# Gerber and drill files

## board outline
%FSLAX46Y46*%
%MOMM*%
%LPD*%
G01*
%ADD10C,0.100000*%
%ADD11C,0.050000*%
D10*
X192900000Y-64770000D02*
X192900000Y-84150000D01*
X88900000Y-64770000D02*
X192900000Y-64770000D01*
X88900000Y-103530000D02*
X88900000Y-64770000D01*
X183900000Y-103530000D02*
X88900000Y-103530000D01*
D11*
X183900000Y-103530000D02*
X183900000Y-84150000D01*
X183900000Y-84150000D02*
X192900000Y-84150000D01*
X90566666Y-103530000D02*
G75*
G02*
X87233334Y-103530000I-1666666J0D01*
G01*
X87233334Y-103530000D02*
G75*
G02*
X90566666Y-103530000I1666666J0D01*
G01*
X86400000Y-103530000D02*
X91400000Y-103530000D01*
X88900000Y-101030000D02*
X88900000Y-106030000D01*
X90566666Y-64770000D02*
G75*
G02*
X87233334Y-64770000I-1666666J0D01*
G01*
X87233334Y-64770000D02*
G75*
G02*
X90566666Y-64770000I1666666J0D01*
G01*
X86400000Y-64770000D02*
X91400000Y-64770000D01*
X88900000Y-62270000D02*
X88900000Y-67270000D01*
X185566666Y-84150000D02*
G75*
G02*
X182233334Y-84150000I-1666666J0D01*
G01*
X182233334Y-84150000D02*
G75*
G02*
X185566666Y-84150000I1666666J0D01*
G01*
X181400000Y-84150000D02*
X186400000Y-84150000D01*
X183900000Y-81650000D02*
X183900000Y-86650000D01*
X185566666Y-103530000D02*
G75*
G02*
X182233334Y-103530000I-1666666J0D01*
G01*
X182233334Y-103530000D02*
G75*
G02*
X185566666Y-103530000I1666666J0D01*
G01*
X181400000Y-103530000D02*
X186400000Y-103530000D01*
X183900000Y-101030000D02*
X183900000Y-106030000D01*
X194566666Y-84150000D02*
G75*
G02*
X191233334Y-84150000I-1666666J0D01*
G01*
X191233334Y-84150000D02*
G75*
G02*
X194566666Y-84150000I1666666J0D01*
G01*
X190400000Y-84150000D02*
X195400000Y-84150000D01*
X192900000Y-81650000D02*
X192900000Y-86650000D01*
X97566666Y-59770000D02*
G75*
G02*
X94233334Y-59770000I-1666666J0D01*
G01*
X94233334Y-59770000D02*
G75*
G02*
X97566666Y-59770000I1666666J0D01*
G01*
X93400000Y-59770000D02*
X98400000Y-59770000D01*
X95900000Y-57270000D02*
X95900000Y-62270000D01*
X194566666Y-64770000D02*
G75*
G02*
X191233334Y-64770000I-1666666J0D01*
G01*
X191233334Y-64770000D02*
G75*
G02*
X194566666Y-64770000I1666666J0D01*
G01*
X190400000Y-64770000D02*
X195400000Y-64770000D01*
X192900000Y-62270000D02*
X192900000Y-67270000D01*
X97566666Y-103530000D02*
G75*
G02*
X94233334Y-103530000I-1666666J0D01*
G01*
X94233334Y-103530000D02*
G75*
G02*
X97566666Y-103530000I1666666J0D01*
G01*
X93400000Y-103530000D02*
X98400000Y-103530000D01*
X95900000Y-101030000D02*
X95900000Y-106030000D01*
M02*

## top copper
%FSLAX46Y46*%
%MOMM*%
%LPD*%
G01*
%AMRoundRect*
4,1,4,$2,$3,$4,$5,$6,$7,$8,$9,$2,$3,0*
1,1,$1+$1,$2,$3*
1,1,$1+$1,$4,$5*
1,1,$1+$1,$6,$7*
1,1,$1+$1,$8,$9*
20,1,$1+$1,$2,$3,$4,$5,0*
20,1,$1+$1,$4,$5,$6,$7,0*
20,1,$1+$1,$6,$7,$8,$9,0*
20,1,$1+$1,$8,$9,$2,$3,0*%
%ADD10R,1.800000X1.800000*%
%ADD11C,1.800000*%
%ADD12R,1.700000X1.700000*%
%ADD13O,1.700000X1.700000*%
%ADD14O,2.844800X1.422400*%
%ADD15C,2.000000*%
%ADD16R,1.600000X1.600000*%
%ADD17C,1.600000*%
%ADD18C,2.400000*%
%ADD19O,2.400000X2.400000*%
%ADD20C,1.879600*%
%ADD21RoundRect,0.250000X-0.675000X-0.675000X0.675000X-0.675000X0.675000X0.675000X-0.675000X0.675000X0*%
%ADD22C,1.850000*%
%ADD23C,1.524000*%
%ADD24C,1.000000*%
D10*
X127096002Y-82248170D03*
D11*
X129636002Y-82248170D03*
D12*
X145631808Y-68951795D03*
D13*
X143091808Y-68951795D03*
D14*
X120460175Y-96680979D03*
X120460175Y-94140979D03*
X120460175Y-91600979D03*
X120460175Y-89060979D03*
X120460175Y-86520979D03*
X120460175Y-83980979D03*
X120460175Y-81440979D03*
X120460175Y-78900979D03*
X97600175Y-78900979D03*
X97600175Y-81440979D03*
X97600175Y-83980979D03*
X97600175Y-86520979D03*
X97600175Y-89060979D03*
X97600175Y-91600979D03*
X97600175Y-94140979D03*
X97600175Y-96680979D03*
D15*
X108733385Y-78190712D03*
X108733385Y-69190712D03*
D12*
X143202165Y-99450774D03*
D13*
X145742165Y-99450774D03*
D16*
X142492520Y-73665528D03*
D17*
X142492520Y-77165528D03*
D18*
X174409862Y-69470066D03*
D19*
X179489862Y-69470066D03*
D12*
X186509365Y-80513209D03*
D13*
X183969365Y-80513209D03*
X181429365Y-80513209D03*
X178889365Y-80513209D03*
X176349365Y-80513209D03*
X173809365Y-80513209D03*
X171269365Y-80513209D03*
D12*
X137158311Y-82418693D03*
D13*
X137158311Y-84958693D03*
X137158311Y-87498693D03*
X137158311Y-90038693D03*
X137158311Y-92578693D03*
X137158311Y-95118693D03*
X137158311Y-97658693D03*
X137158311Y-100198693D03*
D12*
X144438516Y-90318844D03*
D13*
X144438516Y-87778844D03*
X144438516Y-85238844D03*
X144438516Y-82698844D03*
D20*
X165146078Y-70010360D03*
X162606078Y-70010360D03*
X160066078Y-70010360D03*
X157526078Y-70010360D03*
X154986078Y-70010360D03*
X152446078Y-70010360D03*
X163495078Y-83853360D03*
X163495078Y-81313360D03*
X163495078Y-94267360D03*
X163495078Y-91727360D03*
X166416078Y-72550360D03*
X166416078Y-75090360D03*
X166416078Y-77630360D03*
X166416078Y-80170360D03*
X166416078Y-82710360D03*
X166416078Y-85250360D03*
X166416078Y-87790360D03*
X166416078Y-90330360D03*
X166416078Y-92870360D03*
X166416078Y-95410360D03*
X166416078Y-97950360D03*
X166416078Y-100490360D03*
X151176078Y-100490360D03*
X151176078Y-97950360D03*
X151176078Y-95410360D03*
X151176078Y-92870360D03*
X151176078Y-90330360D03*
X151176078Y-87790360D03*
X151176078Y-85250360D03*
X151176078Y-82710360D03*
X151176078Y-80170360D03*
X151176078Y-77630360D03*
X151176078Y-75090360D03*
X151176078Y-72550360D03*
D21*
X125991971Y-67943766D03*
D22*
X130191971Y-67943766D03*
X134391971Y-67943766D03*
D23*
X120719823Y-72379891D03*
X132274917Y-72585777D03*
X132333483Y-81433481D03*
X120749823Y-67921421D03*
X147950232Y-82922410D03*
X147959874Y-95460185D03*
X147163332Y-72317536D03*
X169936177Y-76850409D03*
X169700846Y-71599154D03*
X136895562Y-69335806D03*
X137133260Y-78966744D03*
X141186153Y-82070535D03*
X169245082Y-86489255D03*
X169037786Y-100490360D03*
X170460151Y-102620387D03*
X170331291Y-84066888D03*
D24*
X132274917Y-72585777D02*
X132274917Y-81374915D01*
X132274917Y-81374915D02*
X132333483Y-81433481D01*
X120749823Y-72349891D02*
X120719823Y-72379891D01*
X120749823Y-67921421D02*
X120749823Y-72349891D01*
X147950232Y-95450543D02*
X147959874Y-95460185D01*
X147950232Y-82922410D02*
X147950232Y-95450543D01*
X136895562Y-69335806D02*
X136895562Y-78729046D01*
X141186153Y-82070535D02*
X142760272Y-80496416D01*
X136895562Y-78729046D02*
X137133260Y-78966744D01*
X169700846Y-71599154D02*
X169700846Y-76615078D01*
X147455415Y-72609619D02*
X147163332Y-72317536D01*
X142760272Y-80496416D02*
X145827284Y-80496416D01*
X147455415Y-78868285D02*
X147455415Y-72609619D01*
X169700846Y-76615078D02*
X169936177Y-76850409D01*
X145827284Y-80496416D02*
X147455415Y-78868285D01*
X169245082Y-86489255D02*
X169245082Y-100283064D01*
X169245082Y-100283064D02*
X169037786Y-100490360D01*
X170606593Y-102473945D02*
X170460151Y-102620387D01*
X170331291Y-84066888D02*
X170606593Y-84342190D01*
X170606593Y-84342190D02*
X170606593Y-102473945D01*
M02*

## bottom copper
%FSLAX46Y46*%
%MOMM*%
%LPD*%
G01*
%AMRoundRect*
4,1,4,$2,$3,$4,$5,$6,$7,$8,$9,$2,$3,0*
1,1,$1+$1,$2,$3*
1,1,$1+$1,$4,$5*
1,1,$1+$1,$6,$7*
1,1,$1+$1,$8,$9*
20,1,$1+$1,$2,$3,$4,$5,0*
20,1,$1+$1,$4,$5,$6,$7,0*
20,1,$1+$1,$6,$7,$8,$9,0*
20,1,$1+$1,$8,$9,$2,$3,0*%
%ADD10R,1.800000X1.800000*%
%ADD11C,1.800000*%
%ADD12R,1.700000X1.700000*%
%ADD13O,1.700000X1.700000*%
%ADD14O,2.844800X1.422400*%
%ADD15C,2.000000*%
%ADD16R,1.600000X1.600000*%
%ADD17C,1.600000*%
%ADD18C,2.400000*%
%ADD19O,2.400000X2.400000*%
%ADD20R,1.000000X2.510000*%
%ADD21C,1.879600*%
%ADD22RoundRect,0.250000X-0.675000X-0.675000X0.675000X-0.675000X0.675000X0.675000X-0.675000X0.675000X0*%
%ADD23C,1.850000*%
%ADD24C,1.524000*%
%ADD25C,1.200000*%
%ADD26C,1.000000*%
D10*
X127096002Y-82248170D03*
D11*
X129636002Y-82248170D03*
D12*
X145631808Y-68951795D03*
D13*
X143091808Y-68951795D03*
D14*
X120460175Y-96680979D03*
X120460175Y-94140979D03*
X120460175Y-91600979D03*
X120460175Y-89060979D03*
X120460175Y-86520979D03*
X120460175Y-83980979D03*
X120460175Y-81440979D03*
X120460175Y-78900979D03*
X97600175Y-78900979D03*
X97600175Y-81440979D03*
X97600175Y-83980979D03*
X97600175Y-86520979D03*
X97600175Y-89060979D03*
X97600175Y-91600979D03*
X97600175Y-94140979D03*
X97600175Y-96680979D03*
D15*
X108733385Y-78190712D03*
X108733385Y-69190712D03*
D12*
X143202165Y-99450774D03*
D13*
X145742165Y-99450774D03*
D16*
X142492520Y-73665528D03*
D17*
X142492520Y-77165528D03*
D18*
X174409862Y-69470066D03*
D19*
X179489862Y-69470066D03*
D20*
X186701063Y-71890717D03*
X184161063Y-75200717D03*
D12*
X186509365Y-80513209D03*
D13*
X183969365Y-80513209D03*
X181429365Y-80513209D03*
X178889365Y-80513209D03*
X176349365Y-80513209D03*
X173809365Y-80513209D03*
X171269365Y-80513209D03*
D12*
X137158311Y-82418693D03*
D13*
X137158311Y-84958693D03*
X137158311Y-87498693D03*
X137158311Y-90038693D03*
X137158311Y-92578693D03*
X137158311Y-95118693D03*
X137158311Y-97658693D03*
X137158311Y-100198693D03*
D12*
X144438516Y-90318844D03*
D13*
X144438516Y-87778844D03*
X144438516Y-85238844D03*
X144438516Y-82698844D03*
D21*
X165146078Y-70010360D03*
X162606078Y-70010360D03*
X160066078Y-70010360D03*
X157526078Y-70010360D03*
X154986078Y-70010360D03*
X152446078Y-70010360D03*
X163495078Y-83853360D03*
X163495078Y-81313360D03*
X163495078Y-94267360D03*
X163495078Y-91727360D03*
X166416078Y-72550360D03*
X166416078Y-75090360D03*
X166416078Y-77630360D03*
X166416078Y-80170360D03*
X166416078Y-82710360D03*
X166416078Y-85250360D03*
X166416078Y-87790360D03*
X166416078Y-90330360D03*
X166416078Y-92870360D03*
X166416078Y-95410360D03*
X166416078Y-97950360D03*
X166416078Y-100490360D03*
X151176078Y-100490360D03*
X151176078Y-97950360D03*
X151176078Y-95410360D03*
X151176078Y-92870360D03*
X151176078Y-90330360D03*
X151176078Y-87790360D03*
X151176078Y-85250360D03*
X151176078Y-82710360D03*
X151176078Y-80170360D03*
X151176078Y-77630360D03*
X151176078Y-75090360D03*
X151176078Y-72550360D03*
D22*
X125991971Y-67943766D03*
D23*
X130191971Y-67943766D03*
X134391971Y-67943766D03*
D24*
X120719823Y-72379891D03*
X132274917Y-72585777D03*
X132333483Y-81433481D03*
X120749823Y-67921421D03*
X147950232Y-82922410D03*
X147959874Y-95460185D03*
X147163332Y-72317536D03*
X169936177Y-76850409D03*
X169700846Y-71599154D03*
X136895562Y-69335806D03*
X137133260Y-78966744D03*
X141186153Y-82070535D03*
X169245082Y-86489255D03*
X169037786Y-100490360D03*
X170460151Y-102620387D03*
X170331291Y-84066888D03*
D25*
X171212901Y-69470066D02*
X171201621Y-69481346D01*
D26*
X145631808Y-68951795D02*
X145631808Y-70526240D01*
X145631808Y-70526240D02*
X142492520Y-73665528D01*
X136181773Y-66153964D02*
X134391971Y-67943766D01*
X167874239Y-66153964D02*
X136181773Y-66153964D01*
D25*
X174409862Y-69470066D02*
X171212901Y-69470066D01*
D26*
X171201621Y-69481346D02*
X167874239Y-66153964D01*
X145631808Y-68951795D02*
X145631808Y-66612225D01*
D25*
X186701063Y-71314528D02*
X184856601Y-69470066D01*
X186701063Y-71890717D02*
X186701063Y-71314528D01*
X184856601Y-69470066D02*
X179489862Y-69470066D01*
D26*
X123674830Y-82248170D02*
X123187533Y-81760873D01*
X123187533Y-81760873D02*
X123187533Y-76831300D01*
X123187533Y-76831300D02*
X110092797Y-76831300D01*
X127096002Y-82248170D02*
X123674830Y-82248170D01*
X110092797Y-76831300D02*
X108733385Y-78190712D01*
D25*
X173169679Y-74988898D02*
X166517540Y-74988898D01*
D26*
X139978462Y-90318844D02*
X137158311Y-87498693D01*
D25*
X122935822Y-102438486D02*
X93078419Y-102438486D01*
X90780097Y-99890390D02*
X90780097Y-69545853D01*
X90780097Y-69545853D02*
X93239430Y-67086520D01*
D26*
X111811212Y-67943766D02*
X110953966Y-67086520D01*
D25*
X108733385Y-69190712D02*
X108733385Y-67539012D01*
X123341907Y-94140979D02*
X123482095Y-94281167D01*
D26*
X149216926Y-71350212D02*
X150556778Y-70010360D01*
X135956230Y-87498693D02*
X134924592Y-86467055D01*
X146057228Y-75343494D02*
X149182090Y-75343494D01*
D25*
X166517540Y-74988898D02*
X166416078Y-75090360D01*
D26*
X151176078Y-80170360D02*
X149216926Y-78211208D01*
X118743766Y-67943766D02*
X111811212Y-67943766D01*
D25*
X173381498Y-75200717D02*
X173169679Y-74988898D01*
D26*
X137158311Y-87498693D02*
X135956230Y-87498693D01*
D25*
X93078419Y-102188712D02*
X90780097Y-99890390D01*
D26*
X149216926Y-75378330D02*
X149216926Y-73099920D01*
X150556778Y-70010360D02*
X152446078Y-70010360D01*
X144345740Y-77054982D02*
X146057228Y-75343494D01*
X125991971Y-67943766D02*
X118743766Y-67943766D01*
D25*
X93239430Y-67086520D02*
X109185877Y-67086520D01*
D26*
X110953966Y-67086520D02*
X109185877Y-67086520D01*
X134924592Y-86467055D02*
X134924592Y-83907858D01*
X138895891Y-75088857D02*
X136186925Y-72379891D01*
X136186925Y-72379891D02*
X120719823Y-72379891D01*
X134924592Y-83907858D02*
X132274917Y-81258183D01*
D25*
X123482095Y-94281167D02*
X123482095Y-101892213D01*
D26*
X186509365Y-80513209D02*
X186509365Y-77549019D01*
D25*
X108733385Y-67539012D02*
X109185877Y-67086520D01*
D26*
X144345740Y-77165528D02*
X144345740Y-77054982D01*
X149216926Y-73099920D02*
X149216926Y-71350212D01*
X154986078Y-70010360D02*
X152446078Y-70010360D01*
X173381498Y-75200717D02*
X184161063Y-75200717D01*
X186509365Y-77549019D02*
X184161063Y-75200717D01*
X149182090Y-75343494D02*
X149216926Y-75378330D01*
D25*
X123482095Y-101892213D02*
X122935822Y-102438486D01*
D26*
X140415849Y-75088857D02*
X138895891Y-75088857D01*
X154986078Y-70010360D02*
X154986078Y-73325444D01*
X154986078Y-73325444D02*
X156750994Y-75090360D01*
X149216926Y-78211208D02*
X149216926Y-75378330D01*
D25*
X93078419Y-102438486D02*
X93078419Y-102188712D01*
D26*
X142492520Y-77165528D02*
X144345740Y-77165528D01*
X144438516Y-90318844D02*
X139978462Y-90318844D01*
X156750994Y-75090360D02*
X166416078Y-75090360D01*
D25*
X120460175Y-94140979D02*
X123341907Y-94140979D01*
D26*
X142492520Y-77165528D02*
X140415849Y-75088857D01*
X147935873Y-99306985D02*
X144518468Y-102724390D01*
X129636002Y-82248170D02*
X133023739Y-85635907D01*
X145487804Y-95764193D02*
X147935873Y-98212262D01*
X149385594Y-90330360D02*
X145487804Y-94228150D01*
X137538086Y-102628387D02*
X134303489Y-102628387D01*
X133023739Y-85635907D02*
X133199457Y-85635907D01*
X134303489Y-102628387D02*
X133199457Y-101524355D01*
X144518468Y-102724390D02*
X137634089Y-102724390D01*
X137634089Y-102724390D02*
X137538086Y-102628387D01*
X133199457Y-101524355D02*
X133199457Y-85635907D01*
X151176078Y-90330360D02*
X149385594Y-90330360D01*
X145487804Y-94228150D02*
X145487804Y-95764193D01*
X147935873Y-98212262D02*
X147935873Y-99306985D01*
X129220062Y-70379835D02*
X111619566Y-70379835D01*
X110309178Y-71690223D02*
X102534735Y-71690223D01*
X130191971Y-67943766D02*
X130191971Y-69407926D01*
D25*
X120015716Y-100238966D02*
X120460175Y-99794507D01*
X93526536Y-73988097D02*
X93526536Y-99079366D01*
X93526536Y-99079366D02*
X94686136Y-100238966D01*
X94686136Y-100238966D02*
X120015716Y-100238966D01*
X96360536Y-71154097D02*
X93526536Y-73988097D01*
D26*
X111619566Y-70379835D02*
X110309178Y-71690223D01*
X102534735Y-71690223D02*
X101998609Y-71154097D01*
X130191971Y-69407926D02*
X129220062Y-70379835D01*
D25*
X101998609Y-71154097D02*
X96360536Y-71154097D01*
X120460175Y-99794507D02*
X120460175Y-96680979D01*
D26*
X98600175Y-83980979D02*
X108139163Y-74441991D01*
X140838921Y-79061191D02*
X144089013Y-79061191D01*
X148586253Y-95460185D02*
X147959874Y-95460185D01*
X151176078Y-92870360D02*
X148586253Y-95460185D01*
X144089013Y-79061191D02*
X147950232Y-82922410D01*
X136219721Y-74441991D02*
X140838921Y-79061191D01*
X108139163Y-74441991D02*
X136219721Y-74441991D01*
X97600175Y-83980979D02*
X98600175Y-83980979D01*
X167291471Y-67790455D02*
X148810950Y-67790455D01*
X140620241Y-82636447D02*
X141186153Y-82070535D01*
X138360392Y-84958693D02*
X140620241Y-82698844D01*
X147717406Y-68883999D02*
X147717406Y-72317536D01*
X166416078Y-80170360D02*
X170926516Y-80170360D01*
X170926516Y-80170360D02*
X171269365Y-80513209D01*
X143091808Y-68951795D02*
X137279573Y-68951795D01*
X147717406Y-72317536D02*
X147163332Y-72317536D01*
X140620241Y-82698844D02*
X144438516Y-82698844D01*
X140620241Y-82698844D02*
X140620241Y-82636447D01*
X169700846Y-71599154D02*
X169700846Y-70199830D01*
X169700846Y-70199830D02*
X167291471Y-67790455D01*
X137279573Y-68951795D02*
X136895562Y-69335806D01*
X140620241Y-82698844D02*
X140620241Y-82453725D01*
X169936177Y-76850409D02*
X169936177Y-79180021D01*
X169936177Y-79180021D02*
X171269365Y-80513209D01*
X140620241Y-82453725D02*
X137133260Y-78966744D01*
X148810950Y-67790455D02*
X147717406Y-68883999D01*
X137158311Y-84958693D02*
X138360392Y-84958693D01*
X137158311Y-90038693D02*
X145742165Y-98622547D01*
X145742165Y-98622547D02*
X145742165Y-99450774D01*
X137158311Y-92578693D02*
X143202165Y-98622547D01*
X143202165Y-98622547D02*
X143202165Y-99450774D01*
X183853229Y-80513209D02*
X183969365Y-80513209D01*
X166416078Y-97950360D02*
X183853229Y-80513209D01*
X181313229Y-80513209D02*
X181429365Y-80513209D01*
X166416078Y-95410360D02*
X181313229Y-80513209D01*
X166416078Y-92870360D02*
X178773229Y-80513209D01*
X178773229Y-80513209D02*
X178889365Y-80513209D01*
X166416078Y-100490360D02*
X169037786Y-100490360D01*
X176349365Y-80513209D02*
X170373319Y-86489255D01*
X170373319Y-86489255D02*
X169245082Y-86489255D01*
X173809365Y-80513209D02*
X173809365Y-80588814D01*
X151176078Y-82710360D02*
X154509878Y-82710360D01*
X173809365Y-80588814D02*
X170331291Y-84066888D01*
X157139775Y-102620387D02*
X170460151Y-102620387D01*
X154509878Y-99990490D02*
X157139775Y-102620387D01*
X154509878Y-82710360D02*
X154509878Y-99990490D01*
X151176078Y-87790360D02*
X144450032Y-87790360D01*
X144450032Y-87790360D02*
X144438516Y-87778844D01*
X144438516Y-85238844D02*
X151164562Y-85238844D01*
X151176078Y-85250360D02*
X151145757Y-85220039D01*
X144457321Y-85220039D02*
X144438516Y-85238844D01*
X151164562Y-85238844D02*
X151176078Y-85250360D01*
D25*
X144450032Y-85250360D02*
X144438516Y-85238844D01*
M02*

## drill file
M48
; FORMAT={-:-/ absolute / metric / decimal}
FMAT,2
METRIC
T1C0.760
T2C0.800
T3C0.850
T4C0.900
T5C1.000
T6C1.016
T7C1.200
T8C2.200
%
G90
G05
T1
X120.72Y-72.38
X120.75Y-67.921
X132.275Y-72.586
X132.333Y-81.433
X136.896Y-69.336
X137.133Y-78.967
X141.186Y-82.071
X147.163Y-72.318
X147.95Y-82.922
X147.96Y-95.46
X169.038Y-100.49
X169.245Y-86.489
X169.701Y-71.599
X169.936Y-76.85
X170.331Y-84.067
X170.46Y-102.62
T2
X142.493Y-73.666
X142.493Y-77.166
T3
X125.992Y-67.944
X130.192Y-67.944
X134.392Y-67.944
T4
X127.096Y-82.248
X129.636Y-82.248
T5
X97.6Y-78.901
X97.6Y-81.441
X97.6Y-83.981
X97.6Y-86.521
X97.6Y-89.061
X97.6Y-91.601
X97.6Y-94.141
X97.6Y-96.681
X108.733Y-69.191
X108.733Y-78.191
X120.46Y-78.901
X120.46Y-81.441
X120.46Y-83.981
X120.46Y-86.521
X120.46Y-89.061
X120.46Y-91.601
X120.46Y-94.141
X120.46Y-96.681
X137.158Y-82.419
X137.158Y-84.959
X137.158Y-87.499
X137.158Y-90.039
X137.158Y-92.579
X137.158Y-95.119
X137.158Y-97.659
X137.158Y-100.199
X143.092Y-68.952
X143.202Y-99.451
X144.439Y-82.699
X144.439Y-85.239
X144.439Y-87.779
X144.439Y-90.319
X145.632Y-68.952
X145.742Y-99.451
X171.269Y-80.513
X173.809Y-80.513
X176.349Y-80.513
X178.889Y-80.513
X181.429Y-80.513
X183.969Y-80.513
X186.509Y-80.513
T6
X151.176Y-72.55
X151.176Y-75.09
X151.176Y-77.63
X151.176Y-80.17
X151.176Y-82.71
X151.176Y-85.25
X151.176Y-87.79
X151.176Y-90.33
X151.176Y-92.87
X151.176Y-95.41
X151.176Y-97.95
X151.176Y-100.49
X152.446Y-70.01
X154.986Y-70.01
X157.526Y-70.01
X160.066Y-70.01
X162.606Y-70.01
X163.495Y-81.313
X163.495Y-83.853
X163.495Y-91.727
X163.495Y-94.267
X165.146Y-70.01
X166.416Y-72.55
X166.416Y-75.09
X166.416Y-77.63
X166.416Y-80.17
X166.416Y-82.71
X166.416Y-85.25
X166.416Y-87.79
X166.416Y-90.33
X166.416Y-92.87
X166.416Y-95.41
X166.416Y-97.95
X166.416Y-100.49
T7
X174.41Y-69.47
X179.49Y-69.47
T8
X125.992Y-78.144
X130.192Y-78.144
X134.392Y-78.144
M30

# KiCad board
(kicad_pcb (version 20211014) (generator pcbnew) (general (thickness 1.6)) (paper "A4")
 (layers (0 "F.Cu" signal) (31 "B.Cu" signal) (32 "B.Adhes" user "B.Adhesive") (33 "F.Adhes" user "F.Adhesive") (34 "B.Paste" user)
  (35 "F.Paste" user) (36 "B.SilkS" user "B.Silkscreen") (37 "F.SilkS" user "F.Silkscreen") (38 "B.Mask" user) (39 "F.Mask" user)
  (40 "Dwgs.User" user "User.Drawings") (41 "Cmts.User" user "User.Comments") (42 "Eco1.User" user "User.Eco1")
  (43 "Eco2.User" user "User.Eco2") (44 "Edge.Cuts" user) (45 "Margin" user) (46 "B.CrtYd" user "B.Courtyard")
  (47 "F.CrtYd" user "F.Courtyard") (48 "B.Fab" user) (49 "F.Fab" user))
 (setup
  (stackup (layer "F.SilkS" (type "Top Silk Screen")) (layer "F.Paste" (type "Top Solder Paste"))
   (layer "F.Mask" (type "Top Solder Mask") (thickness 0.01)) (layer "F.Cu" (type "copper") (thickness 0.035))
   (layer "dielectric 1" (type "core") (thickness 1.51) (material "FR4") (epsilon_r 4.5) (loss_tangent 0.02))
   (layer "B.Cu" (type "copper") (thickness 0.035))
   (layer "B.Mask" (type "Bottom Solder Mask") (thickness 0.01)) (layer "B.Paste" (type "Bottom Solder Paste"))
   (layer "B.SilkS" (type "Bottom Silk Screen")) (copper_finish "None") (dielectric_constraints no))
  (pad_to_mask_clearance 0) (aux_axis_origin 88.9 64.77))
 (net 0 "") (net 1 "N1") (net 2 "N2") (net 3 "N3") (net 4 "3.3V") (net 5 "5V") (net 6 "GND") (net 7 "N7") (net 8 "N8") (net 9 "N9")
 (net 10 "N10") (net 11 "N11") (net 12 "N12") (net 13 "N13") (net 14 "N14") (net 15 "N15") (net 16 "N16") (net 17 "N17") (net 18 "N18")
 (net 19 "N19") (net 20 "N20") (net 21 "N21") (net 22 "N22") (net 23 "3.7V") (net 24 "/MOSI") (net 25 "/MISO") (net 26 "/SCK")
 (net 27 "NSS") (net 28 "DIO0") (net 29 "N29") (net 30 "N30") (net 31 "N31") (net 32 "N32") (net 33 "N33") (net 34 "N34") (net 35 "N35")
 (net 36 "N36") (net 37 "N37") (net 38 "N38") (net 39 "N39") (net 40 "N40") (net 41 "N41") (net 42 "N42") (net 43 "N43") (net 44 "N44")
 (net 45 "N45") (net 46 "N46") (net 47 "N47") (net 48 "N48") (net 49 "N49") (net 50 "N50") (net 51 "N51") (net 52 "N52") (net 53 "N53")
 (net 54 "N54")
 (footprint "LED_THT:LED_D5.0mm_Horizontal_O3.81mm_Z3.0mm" (layer "F.Cu") (at 127.096002 82.24817)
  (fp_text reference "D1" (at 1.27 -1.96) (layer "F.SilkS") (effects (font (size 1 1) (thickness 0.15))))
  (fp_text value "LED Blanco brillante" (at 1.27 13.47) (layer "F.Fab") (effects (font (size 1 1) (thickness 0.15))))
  (pad "1" thru_hole rect (at 0 0) (size 1.8 1.8) (drill 0.9) (layers *.Cu *.Mask) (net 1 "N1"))
  (pad "2" thru_hole circle (at 2.54 0) (size 1.8 1.8) (drill 0.9) (layers *.Cu *.Mask) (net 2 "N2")))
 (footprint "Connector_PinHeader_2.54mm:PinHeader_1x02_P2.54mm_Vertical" (layer "F.Cu") (at 145.631808 68.951795 -90)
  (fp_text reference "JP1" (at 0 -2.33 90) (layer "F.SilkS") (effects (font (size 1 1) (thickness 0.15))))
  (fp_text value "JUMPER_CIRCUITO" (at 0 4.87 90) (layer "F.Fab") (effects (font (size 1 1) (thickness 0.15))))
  (pad "1" thru_hole rect (at 0 0 270) (size 1.7 1.7) (drill 1) (layers *.Cu *.Mask) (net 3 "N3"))
  (pad "2" thru_hole oval (at 0 2.54 270) (size 1.7 1.7) (drill 1) (layers *.Cu *.Mask) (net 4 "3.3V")))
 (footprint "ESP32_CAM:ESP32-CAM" (layer "F.Cu") (at 109.030175 86.520979 180)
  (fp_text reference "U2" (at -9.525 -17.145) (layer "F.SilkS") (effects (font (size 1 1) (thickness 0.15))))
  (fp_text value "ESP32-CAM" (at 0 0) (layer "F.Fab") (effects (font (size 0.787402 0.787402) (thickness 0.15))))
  (pad "P$1" thru_hole oval locked (at -11.43 -10.16 180) (size 2.8448 1.4224) (drill 1) (layers *.Cu *.Mask) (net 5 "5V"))
  (pad "P$2" thru_hole oval locked (at -11.43 -7.62 180) (size 2.8448 1.4224) (drill 1) (layers *.Cu *.Mask) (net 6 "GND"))
  (pad "P$3" thru_hole oval locked (at -11.43 -5.08 180) (size 2.8448 1.4224) (drill 1) (layers *.Cu *.Mask) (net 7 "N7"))
  (pad "P$4" thru_hole oval locked (at -11.43 -2.54 180) (size 2.8448 1.4224) (drill 1) (layers *.Cu *.Mask) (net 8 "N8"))
  (pad "P$5" thru_hole oval locked (at -11.43 0 180) (size 2.8448 1.4224) (drill 1) (layers *.Cu *.Mask) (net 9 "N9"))
  (pad "P$6" thru_hole oval locked (at -11.43 2.54 180) (size 2.8448 1.4224) (drill 1) (layers *.Cu *.Mask) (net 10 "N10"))
  (pad "P$7" thru_hole oval locked (at -11.43 5.08 180) (size 2.8448 1.4224) (drill 1) (layers *.Cu *.Mask) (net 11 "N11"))
  (pad "P$8" thru_hole oval locked (at -11.43 7.62 180) (size 2.8448 1.4224) (drill 1) (layers *.Cu *.Mask) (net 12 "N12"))
  (pad "P$9" thru_hole oval locked (at 11.43 7.62 180) (size 2.8448 1.4224) (drill 1) (layers *.Cu *.Mask) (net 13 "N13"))
  (pad "P$10" thru_hole oval locked (at 11.43 5.08 180) (size 2.8448 1.4224) (drill 1) (layers *.Cu *.Mask) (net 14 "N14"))
  (pad "P$11" thru_hole oval locked (at 11.43 2.54 180) (size 2.8448 1.4224) (drill 1) (layers *.Cu *.Mask) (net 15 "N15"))
  (pad "P$12" thru_hole oval locked (at 11.43 0 180) (size 2.8448 1.4224) (drill 1) (layers *.Cu *.Mask) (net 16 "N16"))
  (pad "P$13" thru_hole oval locked (at 11.43 -2.54 180) (size 2.8448 1.4224) (drill 1) (layers *.Cu *.Mask) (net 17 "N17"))
  (pad "P$14" thru_hole oval locked (at 11.43 -5.08 180) (size 2.8448 1.4224) (drill 1) (layers *.Cu *.Mask) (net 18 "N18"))
  (pad "P$15" thru_hole oval locked (at 11.43 -7.62 180) (size 2.8448 1.4224) (drill 1) (layers *.Cu *.Mask) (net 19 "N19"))
  (pad "P$16" thru_hole oval locked (at 11.43 -10.16 180) (size 2.8448 1.4224) (drill 1) (layers *.Cu *.Mask) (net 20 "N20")))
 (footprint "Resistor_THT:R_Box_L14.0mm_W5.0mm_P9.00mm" (layer "F.Cu") (at 108.733385 78.190712 90)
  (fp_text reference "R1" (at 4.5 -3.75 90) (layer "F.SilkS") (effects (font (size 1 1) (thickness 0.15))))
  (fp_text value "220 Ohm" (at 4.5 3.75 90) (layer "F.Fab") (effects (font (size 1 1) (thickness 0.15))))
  (pad "1" thru_hole circle (at 0 0 90) (size 2 2) (drill 1) (layers *.Cu *.Mask) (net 1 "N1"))
  (pad "2" thru_hole circle (at 9 0 90) (size 2 2) (drill 1) (layers *.Cu *.Mask) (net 6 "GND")))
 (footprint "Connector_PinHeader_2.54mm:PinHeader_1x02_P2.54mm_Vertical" (layer "F.Cu") (at 143.202165 99.450774 90)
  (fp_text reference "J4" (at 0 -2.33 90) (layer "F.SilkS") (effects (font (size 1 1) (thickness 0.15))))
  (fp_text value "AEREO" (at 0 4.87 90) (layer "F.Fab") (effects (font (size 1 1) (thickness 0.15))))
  (pad "1" thru_hole rect (at 0 0 90) (size 1.7 1.7) (drill 1) (layers *.Cu *.Mask) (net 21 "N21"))
  (pad "2" thru_hole oval (at 0 2.54 90) (size 1.7 1.7) (drill 1) (layers *.Cu *.Mask) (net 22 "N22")))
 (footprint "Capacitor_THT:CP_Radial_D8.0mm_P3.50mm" (layer "F.Cu") (at 142.49252 73.665528 -90)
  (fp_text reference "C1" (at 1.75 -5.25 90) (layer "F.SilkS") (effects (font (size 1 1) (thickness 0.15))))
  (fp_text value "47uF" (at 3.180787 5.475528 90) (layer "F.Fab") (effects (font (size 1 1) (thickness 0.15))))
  (pad "1" thru_hole rect (at 0 0 270) (size 1.6 1.6) (drill 0.8) (layers *.Cu *.Mask) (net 3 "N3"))
  (pad "2" thru_hole circle (at 3.5 0 270) (size 1.6 1.6) (drill 0.8) (layers *.Cu *.Mask) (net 6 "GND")))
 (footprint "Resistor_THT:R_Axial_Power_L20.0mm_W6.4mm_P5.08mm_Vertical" (layer "F.Cu") (at 174.409862 69.470066)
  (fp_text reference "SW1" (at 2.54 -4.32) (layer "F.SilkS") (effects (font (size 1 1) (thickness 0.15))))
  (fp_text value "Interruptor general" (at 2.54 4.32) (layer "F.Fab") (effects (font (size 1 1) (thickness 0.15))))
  (pad "1" thru_hole circle (at 0 0) (size 2.4 2.4) (drill 1.2) (layers *.Cu *.Mask) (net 3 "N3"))
  (pad "2" thru_hole oval (at 5.08 0) (size 2.4 2.4) (drill 1.2) (layers *.Cu *.Mask) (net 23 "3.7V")))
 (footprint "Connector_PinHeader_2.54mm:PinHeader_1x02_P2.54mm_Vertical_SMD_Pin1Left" (layer "F.Cu") (at 185.431063 73.545717 -90)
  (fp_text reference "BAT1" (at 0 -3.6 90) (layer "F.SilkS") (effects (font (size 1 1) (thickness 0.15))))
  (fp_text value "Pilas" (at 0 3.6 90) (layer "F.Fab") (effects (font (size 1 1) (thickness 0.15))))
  (pad "1" smd rect (at -1.655 -1.27 270) (size 2.51 1) (layers "B.Cu" "F.Paste" "F.Mask") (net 23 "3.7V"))
  (pad "2" smd rect (at 1.655 1.27 270) (size 2.51 1) (layers "B.Cu" "F.Paste" "F.Mask") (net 6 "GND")))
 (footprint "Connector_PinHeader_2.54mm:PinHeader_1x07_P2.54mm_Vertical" (layer "F.Cu") (at 186.509365 80.513209 -90)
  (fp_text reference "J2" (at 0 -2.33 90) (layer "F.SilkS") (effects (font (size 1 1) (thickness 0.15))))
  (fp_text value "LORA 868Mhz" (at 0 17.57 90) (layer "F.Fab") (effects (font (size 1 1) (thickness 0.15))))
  (pad "1" thru_hole rect (at 0 0 270) (size 1.7 1.7) (drill 1) (layers *.Cu *.Mask) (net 6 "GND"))
  (pad "2" thru_hole oval (at 0 2.54 270) (size 1.7 1.7) (drill 1) (layers *.Cu *.Mask) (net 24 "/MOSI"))
  (pad "3" thru_hole oval (at 0 5.08 270) (size 1.7 1.7) (drill 1) (layers *.Cu *.Mask) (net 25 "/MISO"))
  (pad "4" thru_hole oval (at 0 7.62 270) (size 1.7 1.7) (drill 1) (layers *.Cu *.Mask) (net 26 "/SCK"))
  (pad "5" thru_hole oval (at 0 10.16 270) (size 1.7 1.7) (drill 1) (layers *.Cu *.Mask) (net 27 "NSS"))
  (pad "6" thru_hole oval (at 0 12.7 270) (size 1.7 1.7) (drill 1) (layers *.Cu *.Mask) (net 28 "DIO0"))
  (pad "7" thru_hole oval (at 0 15.24 270) (size 1.7 1.7) (drill 1) (layers *.Cu *.Mask) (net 4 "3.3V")))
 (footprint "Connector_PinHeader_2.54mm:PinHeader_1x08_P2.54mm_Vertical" (layer "F.Cu") (at 137.158311 82.418693)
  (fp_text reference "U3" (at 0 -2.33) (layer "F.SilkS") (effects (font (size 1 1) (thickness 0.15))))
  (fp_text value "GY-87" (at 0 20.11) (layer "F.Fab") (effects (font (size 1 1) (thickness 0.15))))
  (pad "1" thru_hole rect (at 0 0) (size 1.7 1.7) (drill 1) (layers *.Cu *.Mask) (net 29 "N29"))
  (pad "2" thru_hole oval (at 0 2.54) (size 1.7 1.7) (drill 1) (layers *.Cu *.Mask) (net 4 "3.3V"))
  (pad "3" thru_hole oval (at 0 5.08) (size 1.7 1.7) (drill 1) (layers *.Cu *.Mask) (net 6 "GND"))
  (pad "4" thru_hole oval (at 0 7.62) (size 1.7 1.7) (drill 1) (layers *.Cu *.Mask) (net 22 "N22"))
  (pad "5" thru_hole oval (at 0 10.16) (size 1.7 1.7) (drill 1) (layers *.Cu *.Mask) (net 21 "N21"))
  (pad "6" thru_hole oval (at 0 12.7) (size 1.7 1.7) (drill 1) (layers *.Cu *.Mask) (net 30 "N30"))
  (pad "7" thru_hole oval (at 0 15.24) (size 1.7 1.7) (drill 1) (layers *.Cu *.Mask) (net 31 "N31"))
  (pad "8" thru_hole oval (at 0 17.78) (size 1.7 1.7) (drill 1) (layers *.Cu *.Mask) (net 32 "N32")))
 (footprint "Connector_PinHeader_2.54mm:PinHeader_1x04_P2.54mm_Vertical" (layer "F.Cu") (at 144.438516 90.318844 180)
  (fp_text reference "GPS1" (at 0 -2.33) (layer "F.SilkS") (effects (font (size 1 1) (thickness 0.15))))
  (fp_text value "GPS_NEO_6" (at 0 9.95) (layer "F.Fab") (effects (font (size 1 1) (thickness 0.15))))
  (pad "1" thru_hole rect (at 0 0 180) (size 1.7 1.7) (drill 1) (layers *.Cu *.Mask) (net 6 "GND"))
  (pad "2" thru_hole oval (at 0 2.54 180) (size 1.7 1.7) (drill 1) (layers *.Cu *.Mask) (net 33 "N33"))
  (pad "3" thru_hole oval (at 0 5.08 180) (size 1.7 1.7) (drill 1) (layers *.Cu *.Mask) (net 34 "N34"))
  (pad "4" thru_hole oval (at 0 7.62 180) (size 1.7 1.7) (drill 1) (layers *.Cu *.Mask) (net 4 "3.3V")))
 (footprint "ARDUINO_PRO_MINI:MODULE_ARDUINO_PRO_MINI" (layer "F.Cu") (at 158.796078 85.25036)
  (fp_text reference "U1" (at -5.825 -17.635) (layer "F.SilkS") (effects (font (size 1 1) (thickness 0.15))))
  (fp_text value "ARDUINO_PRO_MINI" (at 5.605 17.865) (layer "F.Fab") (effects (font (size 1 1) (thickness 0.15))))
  (pad "JP1_1" thru_hole circle locked (at 6.35 -15.24) (size 1.8796 1.8796) (drill 1.016) (layers *.Cu *.Mask) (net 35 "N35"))
  (pad "JP1_2" thru_hole circle locked (at 3.81 -15.24) (size 1.8796 1.8796) (drill 1.016) (layers *.Cu *.Mask) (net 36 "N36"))
  (pad "JP1_3" thru_hole circle locked (at 1.27 -15.24) (size 1.8796 1.8796) (drill 1.016) (layers *.Cu *.Mask) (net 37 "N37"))
  (pad "JP1_4" thru_hole circle locked (at -1.27 -15.24) (size 1.8796 1.8796) (drill 1.016) (layers *.Cu *.Mask) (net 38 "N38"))
  (pad "JP1_5" thru_hole circle locked (at -3.81 -15.24) (size 1.8796 1.8796) (drill 1.016) (layers *.Cu *.Mask) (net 6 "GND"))
  (pad "JP1_6" thru_hole circle locked (at -6.35 -15.24) (size 1.8796 1.8796) (drill 1.016) (layers *.Cu *.Mask) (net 6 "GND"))
  (pad "JP2_1" thru_hole circle locked (at 4.699 -1.397) (size 1.8796 1.8796) (drill 1.016) (layers *.Cu *.Mask) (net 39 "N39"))
  (pad "JP2_2" thru_hole circle locked (at 4.699 -3.937) (size 1.8796 1.8796) (drill 1.016) (layers *.Cu *.Mask) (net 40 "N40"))
  (pad "JP3_1" thru_hole circle locked (at 4.699 9.017) (size 1.8796 1.8796) (drill 1.016) (layers *.Cu *.Mask) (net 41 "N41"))
  (pad "JP3_2" thru_hole circle locked (at 4.699 6.477) (size 1.8796 1.8796) (drill 1.016) (layers *.Cu *.Mask) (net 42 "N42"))
  (pad "JP6_1" thru_hole circle locked (at 7.62 -12.7) (size 1.8796 1.8796) (drill 1.016) (layers *.Cu *.Mask) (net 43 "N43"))
  (pad "JP6_2" thru_hole circle locked (at 7.62 -10.16) (size 1.8796 1.8796) (drill 1.016) (layers *.Cu *.Mask) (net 6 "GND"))
  (pad "JP6_3" thru_hole circle locked (at 7.62 -7.62) (size 1.8796 1.8796) (drill 1.016) (layers *.Cu *.Mask) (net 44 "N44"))
  (pad "JP6_4" thru_hole circle locked (at 7.62 -5.08) (size 1.8796 1.8796) (drill 1.016) (layers *.Cu *.Mask) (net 4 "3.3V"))
  (pad "JP6_5" thru_hole circle locked (at 7.62 -2.54) (size 1.8796 1.8796) (drill 1.016) (layers *.Cu *.Mask) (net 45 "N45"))
  (pad "JP6_6" thru_hole circle locked (at 7.62 0) (size 1.8796 1.8796) (drill 1.016) (layers *.Cu *.Mask) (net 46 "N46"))
  (pad "JP6_7" thru_hole circle locked (at 7.62 2.54) (size 1.8796 1.8796) (drill 1.016) (layers *.Cu *.Mask) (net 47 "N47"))
  (pad "JP6_8" thru_hole circle locked (at 7.62 5.08) (size 1.8796 1.8796) (drill 1.016) (layers *.Cu *.Mask) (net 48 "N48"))
  (pad "JP6_9" thru_hole circle locked (at 7.62 7.62) (size 1.8796 1.8796) (drill 1.016) (layers *.Cu *.Mask) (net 26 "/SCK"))
  (pad "JP6_10" thru_hole circle locked (at 7.62 10.16) (size 1.8796 1.8796) (drill 1.016) (layers *.Cu *.Mask) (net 25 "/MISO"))
  (pad "JP6_11" thru_hole circle locked (at 7.62 12.7) (size 1.8796 1.8796) (drill 1.016) (layers *.Cu *.Mask) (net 24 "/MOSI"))
  (pad "JP6_12" thru_hole circle locked (at 7.62 15.24) (size 1.8796 1.8796) (drill 1.016) (layers *.Cu *.Mask) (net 27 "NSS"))
  (pad "JP7_1" thru_hole circle locked (at -7.62 15.24) (size 1.8796 1.8796) (drill 1.016) (layers *.Cu *.Mask) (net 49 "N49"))
  (pad "JP7_2" thru_hole circle locked (at -7.62 12.7) (size 1.8796 1.8796) (drill 1.016) (layers *.Cu *.Mask) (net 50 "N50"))
  (pad "JP7_3" thru_hole circle locked (at -7.62 10.16) (size 1.8796 1.8796) (drill 1.016) (layers *.Cu *.Mask) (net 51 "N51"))
  (pad "JP7_4" thru_hole circle locked (at -7.62 7.62) (size 1.8796 1.8796) (drill 1.016) (layers *.Cu *.Mask) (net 15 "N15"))
  (pad "JP7_5" thru_hole circle locked (at -7.62 5.08) (size 1.8796 1.8796) (drill 1.016) (layers *.Cu *.Mask) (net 2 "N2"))
  (pad "JP7_6" thru_hole circle locked (at -7.62 2.54) (size 1.8796 1.8796) (drill 1.016) (layers *.Cu *.Mask) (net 33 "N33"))
  (pad "JP7_7" thru_hole circle locked (at -7.62 0) (size 1.8796 1.8796) (drill 1.016) (layers *.Cu *.Mask) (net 34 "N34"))
  (pad "JP7_8" thru_hole circle locked (at -7.62 -2.54) (size 1.8796 1.8796) (drill 1.016) (layers *.Cu *.Mask) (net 28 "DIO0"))
  (pad "JP7_9" thru_hole circle locked (at -7.62 -5.08) (size 1.8796 1.8796) (drill 1.016) (layers *.Cu *.Mask) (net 6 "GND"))
  (pad "JP7_10" thru_hole circle locked (at -7.62 -7.62) (size 1.8796 1.8796) (drill 1.016) (layers *.Cu *.Mask) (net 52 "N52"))
  (pad "JP7_11" thru_hole circle locked (at -7.62 -10.16) (size 1.8796 1.8796) (drill 1.016) (layers *.Cu *.Mask) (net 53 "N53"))
  (pad "JP7_12" thru_hole circle locked (at -7.62 -12.7) (size 1.8796 1.8796) (drill 1.016) (layers *.Cu *.Mask) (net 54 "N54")))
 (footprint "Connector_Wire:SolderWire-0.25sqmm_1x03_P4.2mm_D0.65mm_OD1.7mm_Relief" (layer "F.Cu") (at 125.991971 67.943766)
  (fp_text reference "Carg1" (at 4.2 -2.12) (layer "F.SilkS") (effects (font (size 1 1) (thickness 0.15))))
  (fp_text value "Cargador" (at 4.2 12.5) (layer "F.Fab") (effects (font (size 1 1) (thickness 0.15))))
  (pad "" np_thru_hole circle (at 0 10.2) (size 2.2 2.2) (drill 2.2) (layers *.Cu *.Mask))
  (pad "" np_thru_hole circle (at 8.4 10.2) (size 2.2 2.2) (drill 2.2) (layers *.Cu *.Mask))
  (pad "" np_thru_hole circle (at 4.2 10.2) (size 2.2 2.2) (drill 2.2) (layers *.Cu *.Mask))
  (pad "1" thru_hole roundrect (at 0 0) (size 1.85 1.85) (drill 0.85) (layers *.Cu *.Mask) (roundrect_rratio 0.135135) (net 6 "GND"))
  (pad "2" thru_hole circle (at 4.2 0) (size 1.85 1.85) (drill 0.85) (layers *.Cu *.Mask) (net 5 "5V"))
  (pad "3" thru_hole circle (at 8.4 0) (size 1.85 1.85) (drill 0.85) (layers *.Cu *.Mask) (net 3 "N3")))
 (gr_line (start 192.9 64.77) (end 192.9 84.15) (layer "Edge.Cuts") (width 0.1))
 (gr_line (start 88.9 64.77) (end 192.9 64.77) (layer "Edge.Cuts") (width 0.1))
 (gr_line (start 88.9 103.53) (end 88.9 64.77) (layer "Edge.Cuts") (width 0.1))
 (gr_line (start 183.9 103.53) (end 88.9 103.53) (layer "Edge.Cuts") (width 0.1))
 (gr_line (start 183.9 103.53) (end 183.9 84.15) (layer "Edge.Cuts") (width 0.05))
 (gr_line (start 183.9 84.15) (end 192.9 84.15) (layer "Edge.Cuts") (width 0.05))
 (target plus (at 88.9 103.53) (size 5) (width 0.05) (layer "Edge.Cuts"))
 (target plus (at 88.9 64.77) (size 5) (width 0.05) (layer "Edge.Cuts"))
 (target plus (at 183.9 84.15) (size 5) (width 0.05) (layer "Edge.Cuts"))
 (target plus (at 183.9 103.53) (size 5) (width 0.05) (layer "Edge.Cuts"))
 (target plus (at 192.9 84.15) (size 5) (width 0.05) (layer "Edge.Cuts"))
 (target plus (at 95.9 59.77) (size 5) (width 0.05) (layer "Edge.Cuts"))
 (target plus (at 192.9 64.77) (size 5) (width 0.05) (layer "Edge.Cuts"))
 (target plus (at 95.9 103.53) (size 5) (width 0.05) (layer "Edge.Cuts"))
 (segment (start 171.212901 69.470066) (end 171.201621 69.481346) (width 1.2) (layer "B.Cu") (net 3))
 (segment (start 145.631808 68.951795) (end 145.631808 70.52624) (width 1) (layer "B.Cu") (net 3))
 (segment (start 145.631808 70.52624) (end 142.49252 73.665528) (width 1) (layer "B.Cu") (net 3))
 (segment (start 136.181773 66.153964) (end 134.391971 67.943766) (width 1) (layer "B.Cu") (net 3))
 (segment (start 167.874239 66.153964) (end 136.181773 66.153964) (width 1) (layer "B.Cu") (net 3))
 (segment (start 174.409862 69.470066) (end 171.212901 69.470066) (width 1.2) (layer "B.Cu") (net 3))
 (segment (start 171.201621 69.481346) (end 167.874239 66.153964) (width 1) (layer "B.Cu") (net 3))
 (segment (start 145.631808 68.951795) (end 145.631808 66.612225) (width 1) (layer "B.Cu") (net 3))
 (segment (start 186.701063 71.314528) (end 184.856601 69.470066) (width 1.2) (layer "B.Cu") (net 23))
 (segment (start 186.701063 71.890717) (end 186.701063 71.314528) (width 1.2) (layer "B.Cu") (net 23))
 (segment (start 184.856601 69.470066) (end 179.489862 69.470066) (width 1.2) (layer "B.Cu") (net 23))
 (segment (start 123.67483 82.24817) (end 123.187533 81.760873) (width 1) (layer "B.Cu") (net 1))
 (segment (start 123.187533 81.760873) (end 123.187533 76.8313) (width 1) (layer "B.Cu") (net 1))
 (segment (start 123.187533 76.8313) (end 110.092797 76.8313) (width 1) (layer "B.Cu") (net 1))
 (segment (start 127.096002 82.24817) (end 123.67483 82.24817) (width 1) (layer "B.Cu") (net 1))
 (segment (start 110.092797 76.8313) (end 108.733385 78.190712) (width 1) (layer "B.Cu") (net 1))
 (segment (start 132.274917 72.585777) (end 132.274917 81.374915) (width 1) (layer "F.Cu") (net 6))
 (segment (start 132.274917 81.374915) (end 132.333483 81.433481) (width 1) (layer "F.Cu") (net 6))
 (segment (start 120.749823 72.349891) (end 120.719823 72.379891) (width 1) (layer "F.Cu") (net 6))
 (segment (start 120.749823 67.921421) (end 120.749823 72.349891) (width 1) (layer "F.Cu") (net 6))
 (via (at 120.719823 72.379891) (size 1.524) (drill 0.76) (layers "F.Cu" "B.Cu") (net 6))
 (via (at 132.274917 72.585777) (size 1.524) (drill 0.76) (layers "F.Cu" "B.Cu") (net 6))
 (via (at 132.333483 81.433481) (size 1.524) (drill 0.76) (layers "F.Cu" "B.Cu") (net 6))
 (via (at 120.749823 67.921421) (size 1.524) (drill 0.76) (layers "F.Cu" "B.Cu") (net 6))
 (segment (start 173.169679 74.988898) (end 166.51754 74.988898) (width 1.2) (layer "B.Cu") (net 6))
 (segment (start 139.978462 90.318844) (end 137.158311 87.498693) (width 1) (layer "B.Cu") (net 6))
 (segment (start 122.935822 102.438486) (end 93.078419 102.438486) (width 1.2) (layer "B.Cu") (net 6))
 (segment (start 90.780097 99.89039) (end 90.780097 69.545853) (width 1.2) (layer "B.Cu") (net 6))
 (segment (start 90.780097 69.545853) (end 93.23943 67.08652) (width 1.2) (layer "B.Cu") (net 6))
 (segment (start 111.811212 67.943766) (end 110.953966 67.08652) (width 1) (layer "B.Cu") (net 6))
 (segment (start 108.733385 69.190712) (end 108.733385 67.539012) (width 1.2) (layer "B.Cu") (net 6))
 (segment (start 123.341907 94.140979) (end 123.482095 94.281167) (width 1.2) (layer "B.Cu") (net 6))
 (segment (start 149.216926 71.350212) (end 150.556778 70.01036) (width 1) (layer "B.Cu") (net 6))
 (segment (start 135.95623 87.498693) (end 134.924592 86.467055) (width 1) (layer "B.Cu") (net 6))
 (segment (start 146.057228 75.343494) (end 149.18209 75.343494) (width 1) (layer "B.Cu") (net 6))
 (segment (start 166.51754 74.988898) (end 166.416078 75.09036) (width 1.2) (layer "B.Cu") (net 6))
 (segment (start 151.176078 80.17036) (end 149.216926 78.211208) (width 1) (layer "B.Cu") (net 6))
 (segment (start 118.743766 67.943766) (end 111.811212 67.943766) (width 1) (layer "B.Cu") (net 6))
 (segment (start 173.381498 75.200717) (end 173.169679 74.988898) (width 1.2) (layer "B.Cu") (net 6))
 (segment (start 137.158311 87.498693) (end 135.95623 87.498693) (width 1) (layer "B.Cu") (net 6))
 (segment (start 93.078419 102.188712) (end 90.780097 99.89039) (width 1.2) (layer "B.Cu") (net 6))
 (segment (start 149.216926 75.37833) (end 149.216926 73.09992) (width 1) (layer "B.Cu") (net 6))
 (segment (start 150.556778 70.01036) (end 152.446078 70.01036) (width 1) (layer "B.Cu") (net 6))
 (segment (start 144.34574 77.054982) (end 146.057228 75.343494) (width 1) (layer "B.Cu") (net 6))
 (segment (start 125.991971 67.943766) (end 118.743766 67.943766) (width 1) (layer "B.Cu") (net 6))
 (segment (start 93.23943 67.08652) (end 109.185877 67.08652) (width 1.2) (layer "B.Cu") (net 6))
 (segment (start 110.953966 67.08652) (end 109.185877 67.08652) (width 1) (layer "B.Cu") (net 6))
 (segment (start 134.924592 86.467055) (end 134.924592 83.907858) (width 1) (layer "B.Cu") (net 6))
 (segment (start 138.895891 75.088857) (end 136.186925 72.379891) (width 1) (layer "B.Cu") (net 6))
 (segment (start 136.186925 72.379891) (end 120.719823 72.379891) (width 1) (layer "B.Cu") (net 6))
 (segment (start 134.924592 83.907858) (end 132.274917 81.258183) (width 1) (layer "B.Cu") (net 6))
 (segment (start 123.482095 94.281167) (end 123.482095 101.892213) (width 1.2) (layer "B.Cu") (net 6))
 (segment (start 186.509365 80.513209) (end 186.509365 77.549019) (width 1) (layer "B.Cu") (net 6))
 (segment (start 108.733385 67.539012) (end 109.185877 67.08652) (width 1.2) (layer "B.Cu") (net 6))
 (segment (start 144.34574 77.165528) (end 144.34574 77.054982) (width 1) (layer "B.Cu") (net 6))
 (segment (start 149.216926 73.09992) (end 149.216926 71.350212) (width 1) (layer "B.Cu") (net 6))
 (segment (start 154.986078 70.01036) (end 152.446078 70.01036) (width 1) (layer "B.Cu") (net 6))
 (segment (start 173.381498 75.200717) (end 184.161063 75.200717) (width 1) (layer "B.Cu") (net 6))
 (segment (start 186.509365 77.549019) (end 184.161063 75.200717) (width 1) (layer "B.Cu") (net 6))
 (segment (start 149.18209 75.343494) (end 149.216926 75.37833) (width 1) (layer "B.Cu") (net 6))
 (segment (start 123.482095 101.892213) (end 122.935822 102.438486) (width 1.2) (layer "B.Cu") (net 6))
 (segment (start 140.415849 75.088857) (end 138.895891 75.088857) (width 1) (layer "B.Cu") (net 6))
 (segment (start 154.986078 70.01036) (end 154.986078 73.325444) (width 1) (layer "B.Cu") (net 6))
 (segment (start 154.986078 73.325444) (end 156.750994 75.09036) (width 1) (layer "B.Cu") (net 6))
 (segment (start 149.216926 78.211208) (end 149.216926 75.37833) (width 1) (layer "B.Cu") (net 6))
 (segment (start 93.078419 102.438486) (end 93.078419 102.188712) (width 1.2) (layer "B.Cu") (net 6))
 (segment (start 142.49252 77.165528) (end 144.34574 77.165528) (width 1) (layer "B.Cu") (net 6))
 (segment (start 144.438516 90.318844) (end 139.978462 90.318844) (width 1) (layer "B.Cu") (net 6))
 (segment (start 156.750994 75.09036) (end 166.416078 75.09036) (width 1) (layer "B.Cu") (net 6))
 (segment (start 120.460175 94.140979) (end 123.341907 94.140979) (width 1.2) (layer "B.Cu") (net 6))
 (segment (start 142.49252 77.165528) (end 140.415849 75.088857) (width 1) (layer "B.Cu") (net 6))
 (segment (start 147.935873 99.306985) (end 144.518468 102.72439) (width 1) (layer "B.Cu") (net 2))
 (segment (start 129.636002 82.24817) (end 133.023739 85.635907) (width 1) (layer "B.Cu") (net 2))
 (segment (start 145.487804 95.764193) (end 147.935873 98.212262) (width 1) (layer "B.Cu") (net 2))
 (segment (start 149.385594 90.33036) (end 145.487804 94.22815) (width 1) (layer "B.Cu") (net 2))
 (segment (start 137.538086 102.628387) (end 134.303489 102.628387) (width 1) (layer "B.Cu") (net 2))
 (segment (start 133.023739 85.635907) (end 133.199457 85.635907) (width 1) (layer "B.Cu") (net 2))
 (segment (start 134.303489 102.628387) (end 133.199457 101.524355) (width 1) (layer "B.Cu") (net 2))
 (segment (start 144.518468 102.72439) (end 137.634089 102.72439) (width 1) (layer "B.Cu") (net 2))
 (segment (start 137.634089 102.72439) (end 137.538086 102.628387) (width 1) (layer "B.Cu") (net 2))
 (segment (start 133.199457 101.524355) (end 133.199457 85.635907) (width 1) (layer "B.Cu") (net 2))
 (segment (start 151.176078 90.33036) (end 149.385594 90.33036) (width 1) (layer "B.Cu") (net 2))
 (segment (start 145.487804 94.22815) (end 145.487804 95.764193) (width 1) (layer "B.Cu") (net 2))
 (segment (start 147.935873 98.212262) (end 147.935873 99.306985) (width 1) (layer "B.Cu") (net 2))
 (segment (start 129.220062 70.379835) (end 111.619566 70.379835) (width 1) (layer "B.Cu") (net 5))
 (segment (start 110.309178 71.690223) (end 102.534735 71.690223) (width 1) (layer "B.Cu") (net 5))
 (segment (start 130.191971 67.943766) (end 130.191971 69.407926) (width 1) (layer "B.Cu") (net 5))
 (segment (start 120.015716 100.238966) (end 120.460175 99.794507) (width 1.2) (layer "B.Cu") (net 5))
 (segment (start 93.526536 73.988097) (end 93.526536 99.079366) (width 1.2) (layer "B.Cu") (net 5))
 (segment (start 93.526536 99.079366) (end 94.686136 100.238966) (width 1.2) (layer "B.Cu") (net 5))
 (segment (start 94.686136 100.238966) (end 120.015716 100.238966) (width 1.2) (layer "B.Cu") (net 5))
 (segment (start 96.360536 71.154097) (end 93.526536 73.988097) (width 1.2) (layer "B.Cu") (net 5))
 (segment (start 111.619566 70.379835) (end 110.309178 71.690223) (width 1) (layer "B.Cu") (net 5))
 (segment (start 102.534735 71.690223) (end 101.998609 71.154097) (width 1) (layer "B.Cu") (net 5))
 (segment (start 130.191971 69.407926) (end 129.220062 70.379835) (width 1) (layer "B.Cu") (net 5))
 (segment (start 101.998609 71.154097) (end 96.360536 71.154097) (width 1.2) (layer "B.Cu") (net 5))
 (segment (start 120.460175 99.794507) (end 120.460175 96.680979) (width 1.2) (layer "B.Cu") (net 5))
 (segment (start 147.950232 95.450543) (end 147.959874 95.460185) (width 1) (layer "F.Cu") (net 15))
 (segment (start 147.950232 82.92241) (end 147.950232 95.450543) (width 1) (layer "F.Cu") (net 15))
 (via (at 147.950232 82.92241) (size 1.524) (drill 0.76) (layers "F.Cu" "B.Cu") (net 15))
 (via (at 147.959874 95.460185) (size 1.524) (drill 0.76) (layers "F.Cu" "B.Cu") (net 15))
 (segment (start 98.600175 83.980979) (end 108.139163 74.441991) (width 1) (layer "B.Cu") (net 15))
 (segment (start 140.838921 79.061191) (end 144.089013 79.061191) (width 1) (layer "B.Cu") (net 15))
 (segment (start 148.586253 95.460185) (end 147.959874 95.460185) (width 1) (layer "B.Cu") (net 15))
 (segment (start 151.176078 92.87036) (end 148.586253 95.460185) (width 1) (layer "B.Cu") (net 15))
 (segment (start 144.089013 79.061191) (end 147.950232 82.92241) (width 1) (layer "B.Cu") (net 15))
 (segment (start 136.219721 74.441991) (end 140.838921 79.061191) (width 1) (layer "B.Cu") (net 15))
 (segment (start 108.139163 74.441991) (end 136.219721 74.441991) (width 1) (layer "B.Cu") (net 15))
 (segment (start 97.600175 83.980979) (end 98.600175 83.980979) (width 1) (layer "B.Cu") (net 15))
 (segment (start 136.895562 69.335806) (end 136.895562 78.729046) (width 1) (layer "F.Cu") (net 4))
 (segment (start 141.186153 82.070535) (end 142.760272 80.496416) (width 1) (layer "F.Cu") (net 4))
 (segment (start 136.895562 78.729046) (end 137.13326 78.966744) (width 1) (layer "F.Cu") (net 4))
 (segment (start 169.700846 71.599154) (end 169.700846 76.615078) (width 1) (layer "F.Cu") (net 4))
 (segment (start 147.455415 72.609619) (end 147.163332 72.317536) (width 1) (layer "F.Cu") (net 4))
 (segment (start 142.760272 80.496416) (end 145.827284 80.496416) (width 1) (layer "F.Cu") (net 4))
 (segment (start 147.455415 78.868285) (end 147.455415 72.609619) (width 1) (layer "F.Cu") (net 4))
 (segment (start 169.700846 76.615078) (end 169.936177 76.850409) (width 1) (layer "F.Cu") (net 4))
 (segment (start 145.827284 80.496416) (end 147.455415 78.868285) (width 1) (layer "F.Cu") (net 4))
 (via (at 147.163332 72.317536) (size 1.524) (drill 0.76) (layers "F.Cu" "B.Cu") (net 4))
 (via (at 169.936177 76.850409) (size 1.524) (drill 0.76) (layers "F.Cu" "B.Cu") (free) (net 4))
 (via (at 169.700846 71.599154) (size 1.524) (drill 0.76) (layers "F.Cu" "B.Cu") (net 4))
 (via (at 136.895562 69.335806) (size 1.524) (drill 0.76) (layers "F.Cu" "B.Cu") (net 4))
 (via (at 137.13326 78.966744) (size 1.524) (drill 0.76) (layers "F.Cu" "B.Cu") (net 4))
 (via (at 141.186153 82.070535) (size 1.524) (drill 0.76) (layers "F.Cu" "B.Cu") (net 4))
 (segment (start 167.291471 67.790455) (end 148.81095 67.790455) (width 1) (layer "B.Cu") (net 4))
 (segment (start 140.620241 82.636447) (end 141.186153 82.070535) (width 1) (layer "B.Cu") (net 4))
 (segment (start 138.360392 84.958693) (end 140.620241 82.698844) (width 1) (layer "B.Cu") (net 4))
 (segment (start 147.717406 68.883999) (end 147.717406 72.317536) (width 1) (layer "B.Cu") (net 4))
 (segment (start 166.416078 80.17036) (end 170.926516 80.17036) (width 1) (layer "B.Cu") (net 4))
 (segment (start 170.926516 80.17036) (end 171.269365 80.513209) (width 1) (layer "B.Cu") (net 4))
 (segment (start 143.091808 68.951795) (end 137.279573 68.951795) (width 1) (layer "B.Cu") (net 4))
 (segment (start 147.717406 72.317536) (end 147.163332 72.317536) (width 1) (layer "B.Cu") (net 4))
 (segment (start 140.620241 82.698844) (end 144.438516 82.698844) (width 1) (layer "B.Cu") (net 4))
 (segment (start 140.620241 82.698844) (end 140.620241 82.636447) (width 1) (layer "B.Cu") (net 4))
 (segment (start 169.700846 71.599154) (end 169.700846 70.19983) (width 1) (layer "B.Cu") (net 4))
 (segment (start 169.700846 70.19983) (end 167.291471 67.790455) (width 1) (layer "B.Cu") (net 4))
 (segment (start 137.279573 68.951795) (end 136.895562 69.335806) (width 1) (layer "B.Cu") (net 4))
 (segment (start 140.620241 82.698844) (end 140.620241 82.453725) (width 1) (layer "B.Cu") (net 4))
 (segment (start 169.936177 76.850409) (end 169.936177 79.180021) (width 1) (layer "B.Cu") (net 4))
 (segment (start 169.936177 79.180021) (end 171.269365 80.513209) (width 1) (layer "B.Cu") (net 4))
 (segment (start 140.620241 82.453725) (end 137.13326 78.966744) (width 1) (layer "B.Cu") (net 4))
 (segment (start 148.81095 67.790455) (end 147.717406 68.883999) (width 1) (layer "B.Cu") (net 4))
 (segment (start 137.158311 84.958693) (end 138.360392 84.958693) (width 1) (layer "B.Cu") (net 4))
 (segment (start 137.158311 90.038693) (end 145.742165 98.622547) (width 1) (layer "B.Cu") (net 22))
 (segment (start 145.742165 98.622547) (end 145.742165 99.450774) (width 1) (layer "B.Cu") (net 22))
 (segment (start 137.158311 92.578693) (end 143.202165 98.622547) (width 1) (layer "B.Cu") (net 21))
 (segment (start 143.202165 98.622547) (end 143.202165 99.450774) (width 1) (layer "B.Cu") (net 21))
 (segment (start 183.853229 80.513209) (end 183.969365 80.513209) (width 1) (layer "B.Cu") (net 24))
 (segment (start 166.416078 97.95036) (end 183.853229 80.513209) (width 1) (layer "B.Cu") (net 24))
 (segment (start 181.313229 80.513209) (end 181.429365 80.513209) (width 1) (layer "B.Cu") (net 25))
 (segment (start 166.416078 95.41036) (end 181.313229 80.513209) (width 1) (layer "B.Cu") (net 25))
 (segment (start 166.416078 92.87036) (end 178.773229 80.513209) (width 1) (layer "B.Cu") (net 26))
 (segment (start 178.773229 80.513209) (end 178.889365 80.513209) (width 1) (layer "B.Cu") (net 26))
 (segment (start 169.245082 86.489255) (end 169.245082 100.283064) (width 1) (layer "F.Cu") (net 27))
 (segment (start 169.245082 100.283064) (end 169.037786 100.49036) (width 1) (layer "F.Cu") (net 27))
 (via (at 169.245082 86.489255) (size 1.524) (drill 0.76) (layers "F.Cu" "B.Cu") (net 27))
 (via (at 169.037786 100.49036) (size 1.524) (drill 0.76) (layers "F.Cu" "B.Cu") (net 27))
 (segment (start 166.416078 100.49036) (end 169.037786 100.49036) (width 1) (layer "B.Cu") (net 27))
 (segment (start 176.349365 80.513209) (end 170.373319 86.489255) (width 1) (layer "B.Cu") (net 27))
 (segment (start 170.373319 86.489255) (end 169.245082 86.489255) (width 1) (layer "B.Cu") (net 27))
 (segment (start 170.606593 102.473945) (end 170.460151 102.620387) (width 1) (layer "F.Cu") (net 28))
 (segment (start 170.331291 84.066888) (end 170.606593 84.34219) (width 1) (layer "F.Cu") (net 28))
 (segment (start 170.606593 84.34219) (end 170.606593 102.473945) (width 1) (layer "F.Cu") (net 28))
 (via (at 170.460151 102.620387) (size 1.524) (drill 0.76) (layers "F.Cu" "B.Cu") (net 28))
 (via (at 170.331291 84.066888) (size 1.524) (drill 0.76) (layers "F.Cu" "B.Cu") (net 28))
 (segment (start 173.809365 80.513209) (end 173.809365 80.588814) (width 1) (layer "B.Cu") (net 28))
 (segment (start 151.176078 82.71036) (end 154.509878 82.71036) (width 1) (layer "B.Cu") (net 28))
 (segment (start 173.809365 80.588814) (end 170.331291 84.066888) (width 1) (layer "B.Cu") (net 28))
 (segment (start 157.139775 102.620387) (end 170.460151 102.620387) (width 1) (layer "B.Cu") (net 28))
 (segment (start 154.509878 99.99049) (end 157.139775 102.620387) (width 1) (layer "B.Cu") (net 28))
 (segment (start 154.509878 82.71036) (end 154.509878 99.99049) (width 1) (layer "B.Cu") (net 28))
 (segment (start 151.176078 87.79036) (end 144.450032 87.79036) (width 1) (layer "B.Cu") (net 33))
 (segment (start 144.450032 87.79036) (end 144.438516 87.778844) (width 1) (layer "B.Cu") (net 33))
 (segment (start 144.438516 85.238844) (end 151.164562 85.238844) (width 1) (layer "B.Cu") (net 34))
 (segment (start 151.176078 85.25036) (end 151.145757 85.220039) (width 1) (layer "B.Cu") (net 34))
 (segment (start 144.457321 85.220039) (end 144.438516 85.238844) (width 1) (layer "B.Cu") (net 34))
 (segment (start 151.164562 85.238844) (end 151.176078 85.25036) (width 1) (layer "B.Cu") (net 34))
 (segment (start 144.450032 85.25036) (end 144.438516 85.238844) (width 1.2) (layer "B.Cu") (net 34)))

